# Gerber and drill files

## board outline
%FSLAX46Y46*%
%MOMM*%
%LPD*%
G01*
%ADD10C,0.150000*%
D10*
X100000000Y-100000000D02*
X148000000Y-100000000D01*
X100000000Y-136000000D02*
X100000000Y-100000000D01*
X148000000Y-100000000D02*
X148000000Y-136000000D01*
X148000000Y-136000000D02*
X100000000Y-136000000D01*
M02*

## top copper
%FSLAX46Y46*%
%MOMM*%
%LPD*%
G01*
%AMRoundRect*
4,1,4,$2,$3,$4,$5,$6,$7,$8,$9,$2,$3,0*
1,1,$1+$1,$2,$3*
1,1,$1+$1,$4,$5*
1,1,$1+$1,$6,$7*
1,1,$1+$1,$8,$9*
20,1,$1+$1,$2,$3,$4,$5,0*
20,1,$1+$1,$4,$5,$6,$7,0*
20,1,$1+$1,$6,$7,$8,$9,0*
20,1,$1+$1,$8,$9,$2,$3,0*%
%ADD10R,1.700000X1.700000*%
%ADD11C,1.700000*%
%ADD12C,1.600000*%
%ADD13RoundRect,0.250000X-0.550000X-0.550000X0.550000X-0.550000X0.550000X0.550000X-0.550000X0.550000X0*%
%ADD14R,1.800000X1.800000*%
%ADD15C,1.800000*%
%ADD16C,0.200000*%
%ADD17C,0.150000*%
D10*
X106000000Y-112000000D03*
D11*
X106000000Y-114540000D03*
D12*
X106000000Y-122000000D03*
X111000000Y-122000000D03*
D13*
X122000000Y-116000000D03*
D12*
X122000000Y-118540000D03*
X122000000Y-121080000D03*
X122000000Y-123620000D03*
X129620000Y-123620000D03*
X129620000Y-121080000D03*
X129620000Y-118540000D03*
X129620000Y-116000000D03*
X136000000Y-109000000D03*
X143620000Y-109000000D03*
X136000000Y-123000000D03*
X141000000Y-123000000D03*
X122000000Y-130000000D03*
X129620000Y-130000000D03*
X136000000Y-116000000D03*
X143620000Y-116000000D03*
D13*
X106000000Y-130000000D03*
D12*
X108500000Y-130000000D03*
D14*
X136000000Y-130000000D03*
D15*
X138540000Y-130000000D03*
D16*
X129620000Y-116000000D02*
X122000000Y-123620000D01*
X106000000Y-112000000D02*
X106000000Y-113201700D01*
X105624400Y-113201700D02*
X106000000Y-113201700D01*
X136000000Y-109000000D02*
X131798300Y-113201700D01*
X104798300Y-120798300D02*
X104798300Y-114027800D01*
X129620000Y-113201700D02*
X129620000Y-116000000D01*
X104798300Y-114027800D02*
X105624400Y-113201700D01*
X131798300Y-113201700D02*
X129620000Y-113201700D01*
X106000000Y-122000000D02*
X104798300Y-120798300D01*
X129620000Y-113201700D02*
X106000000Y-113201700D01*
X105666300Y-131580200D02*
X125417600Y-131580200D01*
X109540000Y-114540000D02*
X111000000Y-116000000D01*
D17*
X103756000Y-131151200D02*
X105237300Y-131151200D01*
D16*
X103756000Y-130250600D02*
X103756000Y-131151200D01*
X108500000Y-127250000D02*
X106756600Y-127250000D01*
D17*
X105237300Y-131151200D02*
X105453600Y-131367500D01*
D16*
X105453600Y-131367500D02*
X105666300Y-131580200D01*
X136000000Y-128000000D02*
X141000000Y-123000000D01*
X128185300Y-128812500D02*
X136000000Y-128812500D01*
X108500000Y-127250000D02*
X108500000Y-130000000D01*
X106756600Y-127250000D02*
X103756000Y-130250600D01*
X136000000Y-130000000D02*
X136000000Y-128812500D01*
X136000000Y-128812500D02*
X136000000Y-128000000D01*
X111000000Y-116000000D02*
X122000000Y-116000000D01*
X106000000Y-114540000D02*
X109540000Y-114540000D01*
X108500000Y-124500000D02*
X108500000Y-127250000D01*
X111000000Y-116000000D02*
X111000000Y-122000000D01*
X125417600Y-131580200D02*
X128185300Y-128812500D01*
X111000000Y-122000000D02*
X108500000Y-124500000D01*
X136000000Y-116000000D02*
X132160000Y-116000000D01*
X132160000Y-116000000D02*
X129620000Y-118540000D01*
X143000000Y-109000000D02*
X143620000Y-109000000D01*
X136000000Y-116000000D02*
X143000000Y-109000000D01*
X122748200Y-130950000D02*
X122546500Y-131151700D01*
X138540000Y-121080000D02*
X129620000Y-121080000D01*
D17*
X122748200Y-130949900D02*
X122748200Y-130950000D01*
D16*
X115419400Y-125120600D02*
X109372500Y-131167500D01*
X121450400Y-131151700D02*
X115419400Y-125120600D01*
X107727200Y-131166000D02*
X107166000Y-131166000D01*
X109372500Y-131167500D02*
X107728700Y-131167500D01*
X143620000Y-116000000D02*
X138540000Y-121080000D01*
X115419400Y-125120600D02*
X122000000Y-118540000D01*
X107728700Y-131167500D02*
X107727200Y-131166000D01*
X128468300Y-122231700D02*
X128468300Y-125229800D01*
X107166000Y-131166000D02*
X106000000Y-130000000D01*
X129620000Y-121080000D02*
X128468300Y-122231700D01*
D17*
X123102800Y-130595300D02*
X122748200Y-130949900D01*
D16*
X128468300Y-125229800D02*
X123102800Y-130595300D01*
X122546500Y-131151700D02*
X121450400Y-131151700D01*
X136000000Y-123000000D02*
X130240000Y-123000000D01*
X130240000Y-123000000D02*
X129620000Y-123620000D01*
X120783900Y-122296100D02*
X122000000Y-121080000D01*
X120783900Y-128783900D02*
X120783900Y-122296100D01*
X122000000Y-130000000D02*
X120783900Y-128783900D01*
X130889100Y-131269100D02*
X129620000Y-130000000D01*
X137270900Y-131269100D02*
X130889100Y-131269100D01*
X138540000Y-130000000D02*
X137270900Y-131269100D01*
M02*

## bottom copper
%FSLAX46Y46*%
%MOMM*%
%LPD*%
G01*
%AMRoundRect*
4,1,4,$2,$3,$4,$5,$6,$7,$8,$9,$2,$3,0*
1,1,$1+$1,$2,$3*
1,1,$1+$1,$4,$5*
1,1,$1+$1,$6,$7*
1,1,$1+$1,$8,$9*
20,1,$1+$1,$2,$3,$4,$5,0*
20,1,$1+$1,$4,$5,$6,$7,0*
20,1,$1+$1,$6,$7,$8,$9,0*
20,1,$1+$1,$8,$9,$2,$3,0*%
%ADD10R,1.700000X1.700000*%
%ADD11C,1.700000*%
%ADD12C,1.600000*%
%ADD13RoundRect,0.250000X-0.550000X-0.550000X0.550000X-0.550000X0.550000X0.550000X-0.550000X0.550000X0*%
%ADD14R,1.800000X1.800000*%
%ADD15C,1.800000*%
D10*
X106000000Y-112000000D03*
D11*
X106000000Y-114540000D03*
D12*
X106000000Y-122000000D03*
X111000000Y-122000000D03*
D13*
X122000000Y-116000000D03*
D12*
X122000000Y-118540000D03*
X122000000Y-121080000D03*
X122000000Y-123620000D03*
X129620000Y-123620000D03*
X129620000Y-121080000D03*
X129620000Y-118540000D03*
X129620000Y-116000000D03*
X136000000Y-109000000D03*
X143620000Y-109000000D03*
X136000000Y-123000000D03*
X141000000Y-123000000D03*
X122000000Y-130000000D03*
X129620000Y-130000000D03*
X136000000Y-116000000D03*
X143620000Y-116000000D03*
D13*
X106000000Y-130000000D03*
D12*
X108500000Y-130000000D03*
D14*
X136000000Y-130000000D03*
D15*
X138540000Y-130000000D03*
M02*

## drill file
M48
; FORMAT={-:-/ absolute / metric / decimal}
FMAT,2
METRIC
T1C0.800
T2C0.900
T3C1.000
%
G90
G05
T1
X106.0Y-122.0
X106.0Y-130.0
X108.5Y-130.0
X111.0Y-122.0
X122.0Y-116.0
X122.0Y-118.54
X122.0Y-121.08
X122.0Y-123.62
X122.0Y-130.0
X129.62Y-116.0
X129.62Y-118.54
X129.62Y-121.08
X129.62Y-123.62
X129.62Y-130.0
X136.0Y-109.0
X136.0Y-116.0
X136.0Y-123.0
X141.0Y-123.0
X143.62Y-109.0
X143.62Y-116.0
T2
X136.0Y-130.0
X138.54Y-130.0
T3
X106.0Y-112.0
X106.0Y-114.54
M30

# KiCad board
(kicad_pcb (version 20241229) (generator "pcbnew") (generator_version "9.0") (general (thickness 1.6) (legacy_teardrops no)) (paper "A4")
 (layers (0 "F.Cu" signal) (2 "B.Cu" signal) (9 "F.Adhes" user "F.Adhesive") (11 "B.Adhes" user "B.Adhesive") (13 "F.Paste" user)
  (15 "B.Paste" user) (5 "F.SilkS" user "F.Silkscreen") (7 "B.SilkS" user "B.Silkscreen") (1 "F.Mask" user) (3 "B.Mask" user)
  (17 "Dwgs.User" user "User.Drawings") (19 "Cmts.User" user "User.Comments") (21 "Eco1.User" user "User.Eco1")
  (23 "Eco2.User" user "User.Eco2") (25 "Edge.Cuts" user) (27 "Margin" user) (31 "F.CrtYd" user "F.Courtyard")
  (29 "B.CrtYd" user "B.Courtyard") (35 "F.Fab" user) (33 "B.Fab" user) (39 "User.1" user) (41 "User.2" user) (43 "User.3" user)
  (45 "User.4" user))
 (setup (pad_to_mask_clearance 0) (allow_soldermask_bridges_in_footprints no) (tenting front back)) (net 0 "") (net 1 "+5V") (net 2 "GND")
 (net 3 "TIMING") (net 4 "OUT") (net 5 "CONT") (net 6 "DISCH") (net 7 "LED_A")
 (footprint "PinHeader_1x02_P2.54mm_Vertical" (layer "F.Cu") (at 106 112)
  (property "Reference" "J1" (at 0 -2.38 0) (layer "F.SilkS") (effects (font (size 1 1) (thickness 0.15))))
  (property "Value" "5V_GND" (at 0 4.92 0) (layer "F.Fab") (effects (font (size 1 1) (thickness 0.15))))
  (pad "1" thru_hole rect (at 0 0) (size 1.7 1.7) (drill 1) (layers "*.Cu" "*.Mask") (remove_unused_layers no) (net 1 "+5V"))
  (pad "2" thru_hole circle (at 0 2.54) (size 1.7 1.7) (drill 1) (layers "*.Cu" "*.Mask") (remove_unused_layers no) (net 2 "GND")))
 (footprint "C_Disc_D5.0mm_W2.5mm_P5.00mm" (layer "F.Cu") (at 106 122)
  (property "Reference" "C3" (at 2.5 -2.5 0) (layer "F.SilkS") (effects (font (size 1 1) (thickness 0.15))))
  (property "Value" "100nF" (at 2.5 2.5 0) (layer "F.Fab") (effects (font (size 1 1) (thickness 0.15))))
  (pad "1" thru_hole circle (at 0 0) (size 1.6 1.6) (drill 0.8) (layers "*.Cu" "*.Mask") (remove_unused_layers no) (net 1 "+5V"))
  (pad "2" thru_hole circle (at 5 0) (size 1.6 1.6) (drill 0.8) (layers "*.Cu" "*.Mask") (remove_unused_layers no) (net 2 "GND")))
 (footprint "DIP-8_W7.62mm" (layer "F.Cu") (at 122 116)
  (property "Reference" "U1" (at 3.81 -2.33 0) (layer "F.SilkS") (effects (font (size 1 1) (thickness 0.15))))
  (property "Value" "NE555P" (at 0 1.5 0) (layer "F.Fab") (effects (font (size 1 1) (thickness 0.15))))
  (pad "1" thru_hole roundrect (at 0 0) (size 1.6 1.6) (drill 0.8) (layers "*.Cu" "*.Mask") (remove_unused_layers no)
   (roundrect_rratio 0.15625) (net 2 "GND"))
  (pad "2" thru_hole circle (at 0 2.54) (size 1.6 1.6) (drill 0.8) (layers "*.Cu" "*.Mask") (remove_unused_layers no) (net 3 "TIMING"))
  (pad "3" thru_hole circle (at 0 5.08) (size 1.6 1.6) (drill 0.8) (layers "*.Cu" "*.Mask") (remove_unused_layers no) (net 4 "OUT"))
  (pad "4" thru_hole circle (at 0 7.62) (size 1.6 1.6) (drill 0.8) (layers "*.Cu" "*.Mask") (remove_unused_layers no) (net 1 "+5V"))
  (pad "5" thru_hole circle (at 7.62 7.62) (size 1.6 1.6) (drill 0.8) (layers "*.Cu" "*.Mask") (remove_unused_layers no) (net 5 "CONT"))
  (pad "6" thru_hole circle (at 7.62 5.08) (size 1.6 1.6) (drill 0.8) (layers "*.Cu" "*.Mask") (remove_unused_layers no) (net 3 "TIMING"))
  (pad "7" thru_hole circle (at 7.62 2.54) (size 1.6 1.6) (drill 0.8) (layers "*.Cu" "*.Mask") (remove_unused_layers no) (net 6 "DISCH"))
  (pad "8" thru_hole circle (at 7.62 0) (size 1.6 1.6) (drill 0.8) (layers "*.Cu" "*.Mask") (remove_unused_layers no) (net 1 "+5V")))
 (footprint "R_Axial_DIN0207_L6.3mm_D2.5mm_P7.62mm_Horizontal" (layer "F.Cu") (at 136 109)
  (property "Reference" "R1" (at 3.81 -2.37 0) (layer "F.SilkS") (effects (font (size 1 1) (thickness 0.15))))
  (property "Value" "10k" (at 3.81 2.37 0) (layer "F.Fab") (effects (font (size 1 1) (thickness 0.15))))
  (pad "1" thru_hole circle (at 0 0) (size 1.6 1.6) (drill 0.8) (layers "*.Cu" "*.Mask") (remove_unused_layers no) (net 1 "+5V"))
  (pad "2" thru_hole circle (at 7.62 0) (size 1.6 1.6) (drill 0.8) (layers "*.Cu" "*.Mask") (remove_unused_layers no) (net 6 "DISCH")))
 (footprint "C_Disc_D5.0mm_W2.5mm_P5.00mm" (layer "F.Cu") (at 136 123)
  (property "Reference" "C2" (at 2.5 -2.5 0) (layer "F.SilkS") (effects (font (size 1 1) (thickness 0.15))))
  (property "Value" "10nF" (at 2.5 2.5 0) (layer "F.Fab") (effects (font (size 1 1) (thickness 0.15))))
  (pad "1" thru_hole circle (at 0 0) (size 1.6 1.6) (drill 0.8) (layers "*.Cu" "*.Mask") (remove_unused_layers no) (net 5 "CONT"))
  (pad "2" thru_hole circle (at 5 0) (size 1.6 1.6) (drill 0.8) (layers "*.Cu" "*.Mask") (remove_unused_layers no) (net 2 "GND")))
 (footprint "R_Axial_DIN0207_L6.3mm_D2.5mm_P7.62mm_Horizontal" (layer "F.Cu") (at 122 130)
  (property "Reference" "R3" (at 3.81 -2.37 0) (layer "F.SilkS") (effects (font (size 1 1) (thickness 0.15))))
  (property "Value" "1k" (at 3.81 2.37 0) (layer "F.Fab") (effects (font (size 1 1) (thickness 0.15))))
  (pad "1" thru_hole circle (at 0 0) (size 1.6 1.6) (drill 0.8) (layers "*.Cu" "*.Mask") (remove_unused_layers no) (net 4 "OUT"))
  (pad "2" thru_hole circle (at 7.62 0) (size 1.6 1.6) (drill 0.8) (layers "*.Cu" "*.Mask") (remove_unused_layers no) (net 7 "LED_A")))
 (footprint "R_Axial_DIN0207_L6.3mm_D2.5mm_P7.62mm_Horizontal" (layer "F.Cu") (at 136 116)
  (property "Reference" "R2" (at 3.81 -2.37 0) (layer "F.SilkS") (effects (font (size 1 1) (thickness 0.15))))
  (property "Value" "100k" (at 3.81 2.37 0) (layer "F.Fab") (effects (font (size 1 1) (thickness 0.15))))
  (pad "1" thru_hole circle (at 0 0) (size 1.6 1.6) (drill 0.8) (layers "*.Cu" "*.Mask") (remove_unused_layers no) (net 6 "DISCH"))
  (pad "2" thru_hole circle (at 7.62 0) (size 1.6 1.6) (drill 0.8) (layers "*.Cu" "*.Mask") (remove_unused_layers no) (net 3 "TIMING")))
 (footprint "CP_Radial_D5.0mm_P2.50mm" (layer "F.Cu") (at 106 130)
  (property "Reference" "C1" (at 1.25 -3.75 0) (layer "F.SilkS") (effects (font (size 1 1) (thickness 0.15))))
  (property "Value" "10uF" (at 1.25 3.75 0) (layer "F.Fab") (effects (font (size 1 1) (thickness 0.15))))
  (pad "1" thru_hole roundrect (at 0 0) (size 1.6 1.6) (drill 0.8) (layers "*.Cu" "*.Mask") (remove_unused_layers no)
   (roundrect_rratio 0.15625) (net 3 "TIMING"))
  (pad "2" thru_hole circle (at 2.5 0) (size 1.6 1.6) (drill 0.8) (layers "*.Cu" "*.Mask") (remove_unused_layers no) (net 2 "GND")))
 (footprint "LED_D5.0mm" (layer "F.Cu") (at 136 130)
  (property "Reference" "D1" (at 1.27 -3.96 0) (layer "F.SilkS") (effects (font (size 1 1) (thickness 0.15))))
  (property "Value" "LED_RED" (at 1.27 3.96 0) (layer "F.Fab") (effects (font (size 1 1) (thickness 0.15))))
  (pad "1" thru_hole rect (at 0 0) (size 1.8 1.8) (drill 0.9) (layers "*.Cu" "*.Mask") (remove_unused_layers no) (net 2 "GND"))
  (pad "2" thru_hole circle (at 2.54 0) (size 1.8 1.8) (drill 0.9) (layers "*.Cu" "*.Mask") (remove_unused_layers no) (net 7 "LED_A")))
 (gr_line (start 100 100) (end 148 100) (stroke (width 0.15) (type default)) (layer "Edge.Cuts"))
 (gr_line (start 100 136) (end 100 100) (stroke (width 0.15) (type default)) (layer "Edge.Cuts"))
 (gr_line (start 148 100) (end 148 136) (stroke (width 0.15) (type default)) (layer "Edge.Cuts"))
 (gr_line (start 148 136) (end 100 136) (stroke (width 0.15) (type default)) (layer "Edge.Cuts"))
 (segment (start 129.62 116) (end 122 123.62) (width 0.2) (layer "F.Cu") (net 1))
 (segment (start 106 112) (end 106 113.2017) (width 0.2) (layer "F.Cu") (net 1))
 (segment (start 105.6244 113.2017) (end 106 113.2017) (width 0.2) (layer "F.Cu") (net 1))
 (segment (start 136 109) (end 131.7983 113.2017) (width 0.2) (layer "F.Cu") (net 1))
 (segment (start 104.7983 120.7983) (end 104.7983 114.0278) (width 0.2) (layer "F.Cu") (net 1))
 (segment (start 129.62 113.2017) (end 129.62 116) (width 0.2) (layer "F.Cu") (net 1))
 (segment (start 104.7983 114.0278) (end 105.6244 113.2017) (width 0.2) (layer "F.Cu") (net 1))
 (segment (start 131.7983 113.2017) (end 129.62 113.2017) (width 0.2) (layer "F.Cu") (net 1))
 (segment (start 106 122) (end 104.7983 120.7983) (width 0.2) (layer "F.Cu") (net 1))
 (segment (start 129.62 113.2017) (end 106 113.2017) (width 0.2) (layer "F.Cu") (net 1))
 (segment (start 105.6663 131.5802) (end 125.4176 131.5802) (width 0.2) (layer "F.Cu") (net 2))
 (segment (start 109.54 114.54) (end 111 116) (width 0.2) (layer "F.Cu") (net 2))
 (segment (start 103.756 131.1512) (end 105.2373 131.1512) (width 0.15) (layer "F.Cu") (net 2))
 (segment (start 103.756 130.2506) (end 103.756 131.1512) (width 0.2) (layer "F.Cu") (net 2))
 (segment (start 108.5 127.25) (end 106.7566 127.25) (width 0.2) (layer "F.Cu") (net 2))
 (segment (start 105.2373 131.1512) (end 105.4536 131.3675) (width 0.15) (layer "F.Cu") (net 2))
 (segment (start 105.4536 131.3675) (end 105.6663 131.5802) (width 0.2) (layer "F.Cu") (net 2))
 (segment (start 136 128) (end 141 123) (width 0.2) (layer "F.Cu") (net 2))
 (segment (start 128.1853 128.8125) (end 136 128.8125) (width 0.2) (layer "F.Cu") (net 2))
 (segment (start 108.5 127.25) (end 108.5 130) (width 0.2) (layer "F.Cu") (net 2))
 (segment (start 106.7566 127.25) (end 103.756 130.2506) (width 0.2) (layer "F.Cu") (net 2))
 (segment (start 136 130) (end 136 128.8125) (width 0.2) (layer "F.Cu") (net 2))
 (segment (start 136 128.8125) (end 136 128) (width 0.2) (layer "F.Cu") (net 2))
 (segment (start 111 116) (end 122 116) (width 0.2) (layer "F.Cu") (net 2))
 (segment (start 106 114.54) (end 109.54 114.54) (width 0.2) (layer "F.Cu") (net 2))
 (segment (start 108.5 124.5) (end 108.5 127.25) (width 0.2) (layer "F.Cu") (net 2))
 (segment (start 111 116) (end 111 122) (width 0.2) (layer "F.Cu") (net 2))
 (segment (start 125.4176 131.5802) (end 128.1853 128.8125) (width 0.2) (layer "F.Cu") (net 2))
 (segment (start 111 122) (end 108.5 124.5) (width 0.2) (layer "F.Cu") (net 2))
 (segment (start 136 116) (end 132.16 116) (width 0.2) (layer "F.Cu") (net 6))
 (segment (start 132.16 116) (end 129.62 118.54) (width 0.2) (layer "F.Cu") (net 6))
 (segment (start 143 109) (end 143.62 109) (width 0.2) (layer "F.Cu") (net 6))
 (segment (start 136 116) (end 143 109) (width 0.2) (layer "F.Cu") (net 6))
 (segment (start 122.7482 130.95) (end 122.5465 131.1517) (width 0.2) (layer "F.Cu") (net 3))
 (segment (start 138.54 121.08) (end 129.62 121.08) (width 0.2) (layer "F.Cu") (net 3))
 (segment (start 122.7482 130.9499) (end 122.7482 130.95) (width 0.15) (layer "F.Cu") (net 3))
 (segment (start 115.4194 125.1206) (end 109.3725 131.1675) (width 0.2) (layer "F.Cu") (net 3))
 (segment (start 121.4504 131.1517) (end 115.4194 125.1206) (width 0.2) (layer "F.Cu") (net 3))
 (segment (start 107.7272 131.166) (end 107.166 131.166) (width 0.2) (layer "F.Cu") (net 3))
 (segment (start 109.3725 131.1675) (end 107.7287 131.1675) (width 0.2) (layer "F.Cu") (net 3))
 (segment (start 143.62 116) (end 138.54 121.08) (width 0.2) (layer "F.Cu") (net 3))
 (segment (start 115.4194 125.1206) (end 122 118.54) (width 0.2) (layer "F.Cu") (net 3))
 (segment (start 107.7287 131.1675) (end 107.7272 131.166) (width 0.2) (layer "F.Cu") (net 3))
 (segment (start 128.4683 122.2317) (end 128.4683 125.2298) (width 0.2) (layer "F.Cu") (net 3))
 (segment (start 107.166 131.166) (end 106 130) (width 0.2) (layer "F.Cu") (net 3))
 (segment (start 129.62 121.08) (end 128.4683 122.2317) (width 0.2) (layer "F.Cu") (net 3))
 (segment (start 123.1028 130.5953) (end 122.7482 130.9499) (width 0.15) (layer "F.Cu") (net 3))
 (segment (start 128.4683 125.2298) (end 123.1028 130.5953) (width 0.2) (layer "F.Cu") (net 3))
 (segment (start 122.5465 131.1517) (end 121.4504 131.1517) (width 0.2) (layer "F.Cu") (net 3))
 (segment (start 136 123) (end 130.24 123) (width 0.2) (layer "F.Cu") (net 5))
 (segment (start 130.24 123) (end 129.62 123.62) (width 0.2) (layer "F.Cu") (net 5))
 (segment (start 120.7839 122.2961) (end 122 121.08) (width 0.2) (layer "F.Cu") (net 4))
 (segment (start 120.7839 128.7839) (end 120.7839 122.2961) (width 0.2) (layer "F.Cu") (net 4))
 (segment (start 122 130) (end 120.7839 128.7839) (width 0.2) (layer "F.Cu") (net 4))
 (segment (start 130.8891 131.2691) (end 129.62 130) (width 0.2) (layer "F.Cu") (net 7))
 (segment (start 137.2709 131.2691) (end 130.8891 131.2691) (width 0.2) (layer "F.Cu") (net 7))
 (segment (start 138.54 130) (end 137.2709 131.2691) (width 0.2) (layer "F.Cu") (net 7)))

